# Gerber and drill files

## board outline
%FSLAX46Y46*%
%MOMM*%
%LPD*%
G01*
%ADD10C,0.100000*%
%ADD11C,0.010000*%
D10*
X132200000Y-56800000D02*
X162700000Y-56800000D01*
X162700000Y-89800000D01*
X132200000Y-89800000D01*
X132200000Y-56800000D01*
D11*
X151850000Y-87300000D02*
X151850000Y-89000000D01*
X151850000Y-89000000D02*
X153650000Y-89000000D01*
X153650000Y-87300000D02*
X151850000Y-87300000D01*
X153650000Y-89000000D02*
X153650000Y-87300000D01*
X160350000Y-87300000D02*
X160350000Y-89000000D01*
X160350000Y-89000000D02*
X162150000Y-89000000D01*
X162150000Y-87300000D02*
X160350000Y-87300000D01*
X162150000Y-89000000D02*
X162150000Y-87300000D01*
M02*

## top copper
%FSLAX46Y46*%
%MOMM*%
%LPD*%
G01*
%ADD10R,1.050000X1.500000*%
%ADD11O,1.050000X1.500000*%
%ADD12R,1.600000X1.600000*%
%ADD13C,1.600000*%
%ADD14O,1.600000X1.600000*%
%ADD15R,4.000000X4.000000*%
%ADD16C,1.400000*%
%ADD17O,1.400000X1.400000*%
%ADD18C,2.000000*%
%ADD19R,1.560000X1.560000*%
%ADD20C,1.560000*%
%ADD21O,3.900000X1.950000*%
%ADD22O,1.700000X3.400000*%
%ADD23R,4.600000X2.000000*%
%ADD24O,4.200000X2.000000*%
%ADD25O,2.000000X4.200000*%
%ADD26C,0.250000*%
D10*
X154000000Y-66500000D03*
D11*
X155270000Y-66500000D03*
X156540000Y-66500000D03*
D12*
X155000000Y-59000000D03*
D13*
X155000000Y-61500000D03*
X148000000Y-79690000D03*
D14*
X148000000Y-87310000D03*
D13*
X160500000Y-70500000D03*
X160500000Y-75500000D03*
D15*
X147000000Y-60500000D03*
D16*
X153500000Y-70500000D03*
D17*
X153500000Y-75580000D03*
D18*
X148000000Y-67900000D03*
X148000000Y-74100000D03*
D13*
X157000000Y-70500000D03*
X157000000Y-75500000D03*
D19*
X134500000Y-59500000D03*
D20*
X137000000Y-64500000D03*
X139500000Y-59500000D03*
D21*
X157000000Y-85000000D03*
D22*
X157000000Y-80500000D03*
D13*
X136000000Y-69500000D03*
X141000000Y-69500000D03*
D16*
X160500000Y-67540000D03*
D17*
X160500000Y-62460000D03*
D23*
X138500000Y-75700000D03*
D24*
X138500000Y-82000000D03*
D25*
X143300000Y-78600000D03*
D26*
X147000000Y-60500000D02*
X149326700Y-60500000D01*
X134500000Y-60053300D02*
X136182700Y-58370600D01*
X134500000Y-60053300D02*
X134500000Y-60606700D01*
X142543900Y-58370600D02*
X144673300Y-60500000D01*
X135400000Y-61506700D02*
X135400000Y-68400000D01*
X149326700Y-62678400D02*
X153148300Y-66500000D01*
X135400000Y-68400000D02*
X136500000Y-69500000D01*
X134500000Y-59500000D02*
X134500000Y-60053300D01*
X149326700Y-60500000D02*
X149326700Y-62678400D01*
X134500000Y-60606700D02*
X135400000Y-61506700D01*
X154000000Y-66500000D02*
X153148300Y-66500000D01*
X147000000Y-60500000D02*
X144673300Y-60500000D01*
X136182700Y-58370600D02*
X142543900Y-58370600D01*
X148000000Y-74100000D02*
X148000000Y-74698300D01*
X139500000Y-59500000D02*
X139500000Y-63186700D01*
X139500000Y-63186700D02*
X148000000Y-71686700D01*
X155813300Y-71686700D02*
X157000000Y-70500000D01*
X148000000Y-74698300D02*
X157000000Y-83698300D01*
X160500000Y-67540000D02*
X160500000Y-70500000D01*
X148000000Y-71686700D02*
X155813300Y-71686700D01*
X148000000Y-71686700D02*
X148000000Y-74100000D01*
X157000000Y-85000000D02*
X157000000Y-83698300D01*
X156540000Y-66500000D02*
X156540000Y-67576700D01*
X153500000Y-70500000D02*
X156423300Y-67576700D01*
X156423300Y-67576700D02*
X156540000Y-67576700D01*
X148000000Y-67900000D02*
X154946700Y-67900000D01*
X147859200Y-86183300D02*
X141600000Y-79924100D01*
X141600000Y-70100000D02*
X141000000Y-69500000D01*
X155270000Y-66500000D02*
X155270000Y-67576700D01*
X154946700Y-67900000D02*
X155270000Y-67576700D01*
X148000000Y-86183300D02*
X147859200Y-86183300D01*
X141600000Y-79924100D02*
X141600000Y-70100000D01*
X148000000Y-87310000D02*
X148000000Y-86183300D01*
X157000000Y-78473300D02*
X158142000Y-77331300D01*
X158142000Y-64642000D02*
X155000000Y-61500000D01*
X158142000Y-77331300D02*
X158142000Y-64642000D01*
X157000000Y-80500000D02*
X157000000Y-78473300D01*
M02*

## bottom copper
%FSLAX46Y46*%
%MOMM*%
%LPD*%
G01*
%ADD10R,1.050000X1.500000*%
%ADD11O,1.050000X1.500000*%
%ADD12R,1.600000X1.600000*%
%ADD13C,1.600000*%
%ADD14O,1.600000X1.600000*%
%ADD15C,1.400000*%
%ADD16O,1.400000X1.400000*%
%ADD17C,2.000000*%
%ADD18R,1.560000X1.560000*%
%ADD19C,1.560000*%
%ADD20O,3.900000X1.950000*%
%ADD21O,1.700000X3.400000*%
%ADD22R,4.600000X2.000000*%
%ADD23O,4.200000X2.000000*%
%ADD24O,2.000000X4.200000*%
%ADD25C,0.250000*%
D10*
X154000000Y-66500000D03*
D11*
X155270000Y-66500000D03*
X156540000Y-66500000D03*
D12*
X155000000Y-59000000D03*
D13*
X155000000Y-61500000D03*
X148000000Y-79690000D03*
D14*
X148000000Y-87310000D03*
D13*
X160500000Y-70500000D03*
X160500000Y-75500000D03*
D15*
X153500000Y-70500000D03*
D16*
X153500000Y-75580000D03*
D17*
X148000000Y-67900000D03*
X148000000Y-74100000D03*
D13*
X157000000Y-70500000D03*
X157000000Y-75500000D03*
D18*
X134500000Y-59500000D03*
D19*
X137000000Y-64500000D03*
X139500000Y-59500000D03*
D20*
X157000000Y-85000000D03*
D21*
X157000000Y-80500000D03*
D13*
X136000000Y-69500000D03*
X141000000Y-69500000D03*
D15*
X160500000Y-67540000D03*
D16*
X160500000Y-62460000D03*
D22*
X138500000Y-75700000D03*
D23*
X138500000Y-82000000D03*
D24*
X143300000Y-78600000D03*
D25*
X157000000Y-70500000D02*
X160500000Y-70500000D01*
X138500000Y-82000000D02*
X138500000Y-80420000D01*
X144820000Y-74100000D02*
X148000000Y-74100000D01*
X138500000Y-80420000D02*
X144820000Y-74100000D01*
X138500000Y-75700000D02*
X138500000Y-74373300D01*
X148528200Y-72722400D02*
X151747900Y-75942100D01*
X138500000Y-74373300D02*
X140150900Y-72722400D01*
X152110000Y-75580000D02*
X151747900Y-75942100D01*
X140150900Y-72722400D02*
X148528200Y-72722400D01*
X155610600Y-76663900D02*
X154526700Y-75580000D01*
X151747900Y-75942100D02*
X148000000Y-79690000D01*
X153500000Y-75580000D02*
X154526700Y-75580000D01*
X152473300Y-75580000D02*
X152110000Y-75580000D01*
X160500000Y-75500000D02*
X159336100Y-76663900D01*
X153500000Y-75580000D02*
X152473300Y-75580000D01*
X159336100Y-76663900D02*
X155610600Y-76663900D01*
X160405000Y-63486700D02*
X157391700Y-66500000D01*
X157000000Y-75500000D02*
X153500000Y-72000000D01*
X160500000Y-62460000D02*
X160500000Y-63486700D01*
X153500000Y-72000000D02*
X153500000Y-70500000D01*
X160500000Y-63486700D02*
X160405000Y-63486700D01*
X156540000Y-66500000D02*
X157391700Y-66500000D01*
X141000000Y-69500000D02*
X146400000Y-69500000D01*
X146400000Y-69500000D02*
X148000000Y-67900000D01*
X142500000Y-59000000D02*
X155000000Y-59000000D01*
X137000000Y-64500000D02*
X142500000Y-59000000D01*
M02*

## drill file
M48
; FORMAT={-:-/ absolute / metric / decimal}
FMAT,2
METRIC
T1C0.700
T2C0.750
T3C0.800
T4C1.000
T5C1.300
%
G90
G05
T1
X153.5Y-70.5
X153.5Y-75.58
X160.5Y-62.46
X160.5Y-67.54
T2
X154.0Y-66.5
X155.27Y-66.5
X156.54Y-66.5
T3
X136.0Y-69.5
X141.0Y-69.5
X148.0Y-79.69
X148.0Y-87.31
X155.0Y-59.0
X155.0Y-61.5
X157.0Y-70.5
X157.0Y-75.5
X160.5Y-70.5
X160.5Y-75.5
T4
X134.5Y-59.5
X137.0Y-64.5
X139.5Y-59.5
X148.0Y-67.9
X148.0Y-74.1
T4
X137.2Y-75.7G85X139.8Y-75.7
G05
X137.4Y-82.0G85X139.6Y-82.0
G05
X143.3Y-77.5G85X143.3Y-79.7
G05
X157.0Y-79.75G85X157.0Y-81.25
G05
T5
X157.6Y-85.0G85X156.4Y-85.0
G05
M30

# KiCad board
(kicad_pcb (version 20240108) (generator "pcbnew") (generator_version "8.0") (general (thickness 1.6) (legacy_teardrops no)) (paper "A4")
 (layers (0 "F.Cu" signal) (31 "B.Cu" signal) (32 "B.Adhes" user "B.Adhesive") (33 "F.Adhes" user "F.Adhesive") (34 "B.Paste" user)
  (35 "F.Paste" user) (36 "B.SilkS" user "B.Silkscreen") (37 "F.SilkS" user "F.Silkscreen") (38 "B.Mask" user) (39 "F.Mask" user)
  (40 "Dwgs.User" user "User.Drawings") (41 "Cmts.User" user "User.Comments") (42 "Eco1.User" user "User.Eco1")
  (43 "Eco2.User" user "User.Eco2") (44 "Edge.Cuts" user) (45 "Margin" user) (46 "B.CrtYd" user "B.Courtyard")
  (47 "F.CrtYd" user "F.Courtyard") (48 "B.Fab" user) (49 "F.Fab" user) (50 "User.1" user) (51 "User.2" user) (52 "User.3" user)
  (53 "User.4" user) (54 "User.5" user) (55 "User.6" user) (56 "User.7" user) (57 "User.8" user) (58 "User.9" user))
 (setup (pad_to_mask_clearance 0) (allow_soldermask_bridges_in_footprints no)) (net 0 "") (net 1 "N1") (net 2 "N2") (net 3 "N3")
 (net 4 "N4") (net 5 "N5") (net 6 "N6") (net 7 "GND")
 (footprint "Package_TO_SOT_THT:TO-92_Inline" (layer "F.Cu") (at 154 66.5)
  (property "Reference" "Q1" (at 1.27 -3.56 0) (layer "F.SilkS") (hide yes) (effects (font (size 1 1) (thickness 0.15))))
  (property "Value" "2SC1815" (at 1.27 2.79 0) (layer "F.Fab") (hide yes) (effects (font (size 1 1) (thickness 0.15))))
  (pad "1" thru_hole rect (at 0 0) (size 1.05 1.5) (drill 0.75) (layers "*.Cu" "*.Mask") (remove_unused_layers no) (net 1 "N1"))
  (pad "2" thru_hole oval (at 1.27 0) (size 1.05 1.5) (drill 0.75) (layers "*.Cu" "*.Mask") (remove_unused_layers no) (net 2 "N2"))
  (pad "3" thru_hole oval (at 2.54 0) (size 1.05 1.5) (drill 0.75) (layers "*.Cu" "*.Mask") (remove_unused_layers no) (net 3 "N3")))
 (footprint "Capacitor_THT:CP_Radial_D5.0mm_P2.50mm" (layer "F.Cu") (at 155 59 -90)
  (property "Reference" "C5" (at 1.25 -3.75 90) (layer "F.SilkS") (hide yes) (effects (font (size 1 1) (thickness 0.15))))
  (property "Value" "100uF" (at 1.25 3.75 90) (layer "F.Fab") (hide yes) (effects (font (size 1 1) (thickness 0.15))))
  (pad "1" thru_hole rect (at 0 0 270) (size 1.6 1.6) (drill 0.8) (layers "*.Cu" "*.Mask") (remove_unused_layers no) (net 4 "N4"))
  (pad "2" thru_hole circle (at 2.5 0 270) (size 1.6 1.6) (drill 0.8) (layers "*.Cu" "*.Mask") (remove_unused_layers no) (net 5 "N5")))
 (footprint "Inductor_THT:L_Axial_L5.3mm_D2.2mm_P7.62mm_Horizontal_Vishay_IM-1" (layer "F.Cu") (at 148 79.69 -90)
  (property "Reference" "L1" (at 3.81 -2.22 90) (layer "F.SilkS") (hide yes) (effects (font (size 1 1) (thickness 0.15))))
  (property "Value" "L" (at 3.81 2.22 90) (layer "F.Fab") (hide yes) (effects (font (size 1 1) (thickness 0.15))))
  (pad "1" thru_hole circle (at 0 0 270) (size 1.6 1.6) (drill 0.8) (layers "*.Cu" "*.Mask") (remove_unused_layers no) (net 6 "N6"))
  (pad "2" thru_hole oval (at 7.62 0 270) (size 1.6 1.6) (drill 0.8) (layers "*.Cu" "*.Mask") (remove_unused_layers no) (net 2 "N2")))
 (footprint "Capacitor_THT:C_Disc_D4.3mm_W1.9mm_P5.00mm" (layer "F.Cu") (at 160.5 70.5 -90)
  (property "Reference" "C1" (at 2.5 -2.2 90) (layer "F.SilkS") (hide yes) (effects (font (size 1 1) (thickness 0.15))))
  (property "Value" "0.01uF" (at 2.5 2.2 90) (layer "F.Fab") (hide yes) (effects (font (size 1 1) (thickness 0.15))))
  (pad "1" thru_hole circle (at 0 0 270) (size 1.6 1.6) (drill 0.8) (layers "*.Cu" "*.Mask") (remove_unused_layers no) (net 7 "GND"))
  (pad "2" thru_hole circle (at 5 0 270) (size 1.6 1.6) (drill 0.8) (layers "*.Cu" "*.Mask") (remove_unused_layers no) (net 6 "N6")))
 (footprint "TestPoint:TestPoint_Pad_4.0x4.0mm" (layer "F.Cu") (at 147 60.5)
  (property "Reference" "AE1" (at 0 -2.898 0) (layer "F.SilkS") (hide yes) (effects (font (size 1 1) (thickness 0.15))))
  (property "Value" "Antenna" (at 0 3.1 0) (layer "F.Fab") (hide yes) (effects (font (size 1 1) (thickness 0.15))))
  (pad "1" smd rect (at 0 0) (size 4 4) (layers "F.Cu" "F.Mask") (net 1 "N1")))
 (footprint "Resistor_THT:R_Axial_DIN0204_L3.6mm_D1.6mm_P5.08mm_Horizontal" (layer "F.Cu") (at 153.5 70.5 -90)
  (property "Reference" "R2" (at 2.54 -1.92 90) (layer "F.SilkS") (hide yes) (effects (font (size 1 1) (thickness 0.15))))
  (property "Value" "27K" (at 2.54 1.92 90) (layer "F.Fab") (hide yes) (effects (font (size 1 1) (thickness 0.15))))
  (pad "1" thru_hole circle (at 0 0 270) (size 1.4 1.4) (drill 0.7) (layers "*.Cu" "*.Mask") (remove_unused_layers no) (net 3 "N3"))
  (pad "2" thru_hole oval (at 5.08 0 270) (size 1.4 1.4) (drill 0.7) (layers "*.Cu" "*.Mask") (remove_unused_layers no) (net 6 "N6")))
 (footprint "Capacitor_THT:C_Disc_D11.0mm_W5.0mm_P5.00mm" (layer "F.Cu") (at 148 68.4 -90)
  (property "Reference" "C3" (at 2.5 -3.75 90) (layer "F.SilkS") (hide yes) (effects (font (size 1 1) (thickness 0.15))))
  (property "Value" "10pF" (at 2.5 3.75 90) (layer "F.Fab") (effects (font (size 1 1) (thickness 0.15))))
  (pad "1" thru_hole circle (at -0.5 0 270) (size 2 2) (drill 1) (layers "*.Cu" "*.Mask") (remove_unused_layers no) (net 2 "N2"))
  (pad "2" thru_hole circle (at 5.7 0 270) (size 2 2) (drill 1) (layers "*.Cu" "*.Mask") (remove_unused_layers no) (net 7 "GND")))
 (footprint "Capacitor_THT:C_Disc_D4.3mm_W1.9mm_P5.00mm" (layer "F.Cu") (at 157 70.5 -90)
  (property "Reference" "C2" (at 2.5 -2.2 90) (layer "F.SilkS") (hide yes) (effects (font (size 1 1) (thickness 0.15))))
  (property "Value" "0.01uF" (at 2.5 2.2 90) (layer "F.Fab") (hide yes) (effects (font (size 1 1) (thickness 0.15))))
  (pad "1" thru_hole circle (at 0 0 270) (size 1.6 1.6) (drill 0.8) (layers "*.Cu" "*.Mask") (remove_unused_layers no) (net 7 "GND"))
  (pad "2" thru_hole circle (at 5 0 270) (size 1.6 1.6) (drill 0.8) (layers "*.Cu" "*.Mask") (remove_unused_layers no) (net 3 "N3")))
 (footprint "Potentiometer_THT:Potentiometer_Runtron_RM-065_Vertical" (layer "F.Cu") (at 134.5 59.5)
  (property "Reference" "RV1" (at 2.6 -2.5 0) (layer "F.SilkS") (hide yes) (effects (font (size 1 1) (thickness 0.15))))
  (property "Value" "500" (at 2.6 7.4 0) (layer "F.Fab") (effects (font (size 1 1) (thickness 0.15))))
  (pad "1" thru_hole rect (at 0 0) (size 1.56 1.56) (drill 1) (layers "*.Cu" "*.Mask") (remove_unused_layers no) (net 1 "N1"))
  (pad "2" thru_hole circle (at 2.5 5) (size 1.56 1.56) (drill 1) (layers "*.Cu" "*.Mask") (remove_unused_layers no) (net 4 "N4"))
  (pad "3" thru_hole circle (at 5 0) (size 1.56 1.56) (drill 1) (layers "*.Cu" "*.Mask") (remove_unused_layers no) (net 7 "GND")))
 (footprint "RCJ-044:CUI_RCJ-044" (layer "F.Cu") (at 157 85 -90)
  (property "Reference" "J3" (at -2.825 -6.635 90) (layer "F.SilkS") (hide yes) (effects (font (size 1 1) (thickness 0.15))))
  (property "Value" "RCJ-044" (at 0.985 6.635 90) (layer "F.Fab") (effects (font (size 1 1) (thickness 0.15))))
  (fp_line (start 2.3 5.15) (end 4 5.15) (stroke (width 0.01) (type solid)) (layer "Edge.Cuts"))
  (fp_line (start 4 5.15) (end 4 3.35) (stroke (width 0.01) (type solid)) (layer "Edge.Cuts"))
  (fp_line (start 2.3 3.35) (end 2.3 5.15) (stroke (width 0.01) (type solid)) (layer "Edge.Cuts"))
  (fp_line (start 4 3.35) (end 2.3 3.35) (stroke (width 0.01) (type solid)) (layer "Edge.Cuts"))
  (fp_line (start 2.3 -3.35) (end 4 -3.35) (stroke (width 0.01) (type solid)) (layer "Edge.Cuts"))
  (fp_line (start 4 -3.35) (end 4 -5.15) (stroke (width 0.01) (type solid)) (layer "Edge.Cuts"))
  (fp_line (start 2.3 -5.15) (end 2.3 -3.35) (stroke (width 0.01) (type solid)) (layer "Edge.Cuts"))
  (fp_line (start 4 -5.15) (end 2.3 -5.15) (stroke (width 0.01) (type solid)) (layer "Edge.Cuts"))
  (pad "1" thru_hole oval (at 0 0 270) (size 1.95 3.9) (drill oval 1.3 2.5) (layers "*.Cu" "*.Mask") (remove_unused_layers no) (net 7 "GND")
   (solder_mask_margin 0.102))
  (pad "2" thru_hole oval (at -4.5 0 270) (size 3.4 1.7) (drill oval 2.5 1) (layers "*.Cu" "*.Mask") (remove_unused_layers no) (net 5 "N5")
   (solder_mask_margin 0.102)))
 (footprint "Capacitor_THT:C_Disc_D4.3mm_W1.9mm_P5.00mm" (layer "F.Cu") (at 136 69.5)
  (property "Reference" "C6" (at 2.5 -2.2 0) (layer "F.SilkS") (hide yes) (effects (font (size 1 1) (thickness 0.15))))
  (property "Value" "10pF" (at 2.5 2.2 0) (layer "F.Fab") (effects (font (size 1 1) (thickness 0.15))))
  (pad "1" thru_hole circle (at 0 0) (size 1.6 1.6) (drill 0.8) (layers "*.Cu" "*.Mask") (remove_unused_layers no) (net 1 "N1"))
  (pad "2" thru_hole circle (at 5 0) (size 1.6 1.6) (drill 0.8) (layers "*.Cu" "*.Mask") (remove_unused_layers no) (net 2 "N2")))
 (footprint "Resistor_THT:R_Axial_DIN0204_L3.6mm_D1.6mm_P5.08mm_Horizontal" (layer "F.Cu") (at 160.5 67.54 90)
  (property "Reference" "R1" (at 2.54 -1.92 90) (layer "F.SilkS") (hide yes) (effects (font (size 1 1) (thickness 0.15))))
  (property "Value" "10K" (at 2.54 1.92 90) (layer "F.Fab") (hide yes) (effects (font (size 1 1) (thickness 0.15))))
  (pad "1" thru_hole circle (at 0 0 90) (size 1.4 1.4) (drill 0.7) (layers "*.Cu" "*.Mask") (remove_unused_layers no) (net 7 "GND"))
  (pad "2" thru_hole oval (at 5.08 0 90) (size 1.4 1.4) (drill 0.7) (layers "*.Cu" "*.Mask") (remove_unused_layers no) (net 3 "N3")))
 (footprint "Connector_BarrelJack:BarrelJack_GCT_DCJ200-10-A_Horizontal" (layer "F.Cu") (at 138.5 75.7)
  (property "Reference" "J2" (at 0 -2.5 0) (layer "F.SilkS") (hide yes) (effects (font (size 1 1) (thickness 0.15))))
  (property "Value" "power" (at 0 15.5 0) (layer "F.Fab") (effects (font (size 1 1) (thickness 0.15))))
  (pad "1" thru_hole rect (at 0 0) (size 4.6 2) (drill oval 3.6 1) (layers "*.Cu" "*.Mask") (remove_unused_layers no) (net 6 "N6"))
  (pad "2" thru_hole oval (at 0 6.3) (size 4.2 2) (drill oval 3.2 1) (layers "*.Cu" "*.Mask") (remove_unused_layers no) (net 7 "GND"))
  (pad "3" thru_hole oval (at 4.8 2.9) (size 2 4.2) (drill oval 1 3.2) (layers "*.Cu" "*.Mask") (remove_unused_layers no)))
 (gr_rect (start 132.2 56.8) (end 162.7 89.8) (stroke (width 0.1) (type solid)) (fill none) (layer "Edge.Cuts"))
 (segment (start 147 60.5) (end 149.3267 60.5) (width 0.25) (layer "F.Cu") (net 1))
 (segment (start 134.5 60.0533) (end 136.1827 58.3706) (width 0.25) (layer "F.Cu") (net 1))
 (segment (start 134.5 60.0533) (end 134.5 60.6067) (width 0.25) (layer "F.Cu") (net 1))
 (segment (start 142.5439 58.3706) (end 144.6733 60.5) (width 0.25) (layer "F.Cu") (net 1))
 (segment (start 135.4 61.5067) (end 135.4 68.4) (width 0.25) (layer "F.Cu") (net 1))
 (segment (start 149.3267 62.6784) (end 153.1483 66.5) (width 0.25) (layer "F.Cu") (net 1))
 (segment (start 135.4 68.4) (end 136.5 69.5) (width 0.25) (layer "F.Cu") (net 1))
 (segment (start 134.5 59.5) (end 134.5 60.0533) (width 0.25) (layer "F.Cu") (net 1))
 (segment (start 149.3267 60.5) (end 149.3267 62.6784) (width 0.25) (layer "F.Cu") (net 1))
 (segment (start 134.5 60.6067) (end 135.4 61.5067) (width 0.25) (layer "F.Cu") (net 1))
 (segment (start 154 66.5) (end 153.1483 66.5) (width 0.25) (layer "F.Cu") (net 1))
 (segment (start 147 60.5) (end 144.6733 60.5) (width 0.25) (layer "F.Cu") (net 1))
 (segment (start 136.1827 58.3706) (end 142.5439 58.3706) (width 0.25) (layer "F.Cu") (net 1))
 (segment (start 148 74.1) (end 148 74.6983) (width 0.25) (layer "F.Cu") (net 7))
 (segment (start 139.5 59.5) (end 139.5 63.1867) (width 0.25) (layer "F.Cu") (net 7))
 (segment (start 139.5 63.1867) (end 148 71.6867) (width 0.25) (layer "F.Cu") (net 7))
 (segment (start 155.8133 71.6867) (end 157 70.5) (width 0.25) (layer "F.Cu") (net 7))
 (segment (start 148 74.6983) (end 157 83.6983) (width 0.25) (layer "F.Cu") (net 7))
 (segment (start 160.5 67.54) (end 160.5 70.5) (width 0.25) (layer "F.Cu") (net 7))
 (segment (start 148 71.6867) (end 155.8133 71.6867) (width 0.25) (layer "F.Cu") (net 7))
 (segment (start 148 71.6867) (end 148 74.1) (width 0.25) (layer "F.Cu") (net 7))
 (segment (start 157 85) (end 157 83.6983) (width 0.25) (layer "F.Cu") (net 7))
 (segment (start 157 70.5) (end 160.5 70.5) (width 0.25) (layer "B.Cu") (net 7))
 (segment (start 138.5 82) (end 138.5 80.42) (width 0.25) (layer "B.Cu") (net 7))
 (segment (start 144.82 74.1) (end 148 74.1) (width 0.25) (layer "B.Cu") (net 7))
 (segment (start 138.5 80.42) (end 144.82 74.1) (width 0.25) (layer "B.Cu") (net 7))
 (segment (start 138.5 75.7) (end 138.5 74.3733) (width 0.25) (layer "B.Cu") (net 6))
 (segment (start 148.5282 72.7224) (end 151.7479 75.9421) (width 0.25) (layer "B.Cu") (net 6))
 (segment (start 138.5 74.3733) (end 140.1509 72.7224) (width 0.25) (layer "B.Cu") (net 6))
 (segment (start 152.11 75.58) (end 151.7479 75.9421) (width 0.25) (layer "B.Cu") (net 6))
 (segment (start 140.1509 72.7224) (end 148.5282 72.7224) (width 0.25) (layer "B.Cu") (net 6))
 (segment (start 155.6106 76.6639) (end 154.5267 75.58) (width 0.25) (layer "B.Cu") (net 6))
 (segment (start 151.7479 75.9421) (end 148 79.69) (width 0.25) (layer "B.Cu") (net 6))
 (segment (start 153.5 75.58) (end 154.5267 75.58) (width 0.25) (layer "B.Cu") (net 6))
 (segment (start 152.4733 75.58) (end 152.11 75.58) (width 0.25) (layer "B.Cu") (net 6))
 (segment (start 160.5 75.5) (end 159.3361 76.6639) (width 0.25) (layer "B.Cu") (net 6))
 (segment (start 153.5 75.58) (end 152.4733 75.58) (width 0.25) (layer "B.Cu") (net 6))
 (segment (start 159.3361 76.6639) (end 155.6106 76.6639) (width 0.25) (layer "B.Cu") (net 6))
 (segment (start 156.54 66.5) (end 156.54 67.5767) (width 0.25) (layer "F.Cu") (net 3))
 (segment (start 153.5 70.5) (end 156.4233 67.5767) (width 0.25) (layer "F.Cu") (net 3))
 (segment (start 156.4233 67.5767) (end 156.54 67.5767) (width 0.25) (layer "F.Cu") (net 3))
 (segment (start 160.405 63.4867) (end 157.3917 66.5) (width 0.25) (layer "B.Cu") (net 3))
 (segment (start 157 75.5) (end 153.5 72) (width 0.25) (layer "B.Cu") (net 3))
 (segment (start 160.5 62.46) (end 160.5 63.4867) (width 0.25) (layer "B.Cu") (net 3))
 (segment (start 153.5 72) (end 153.5 70.5) (width 0.25) (layer "B.Cu") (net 3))
 (segment (start 160.5 63.4867) (end 160.405 63.4867) (width 0.25) (layer "B.Cu") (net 3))
 (segment (start 156.54 66.5) (end 157.3917 66.5) (width 0.25) (layer "B.Cu") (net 3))
 (segment (start 148 67.9) (end 154.9467 67.9) (width 0.25) (layer "F.Cu") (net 2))
 (segment (start 147.8592 86.1833) (end 141.6 79.9241) (width 0.25) (layer "F.Cu") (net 2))
 (segment (start 141.6 70.1) (end 141 69.5) (width 0.25) (layer "F.Cu") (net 2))
 (segment (start 155.27 66.5) (end 155.27 67.5767) (width 0.25) (layer "F.Cu") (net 2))
 (segment (start 154.9467 67.9) (end 155.27 67.5767) (width 0.25) (layer "F.Cu") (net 2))
 (segment (start 148 86.1833) (end 147.8592 86.1833) (width 0.25) (layer "F.Cu") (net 2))
 (segment (start 141.6 79.9241) (end 141.6 70.1) (width 0.25) (layer "F.Cu") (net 2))
 (segment (start 148 87.31) (end 148 86.1833) (width 0.25) (layer "F.Cu") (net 2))
 (segment (start 141 69.5) (end 146.4 69.5) (width 0.25) (layer "B.Cu") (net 2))
 (segment (start 146.4 69.5) (end 148 67.9) (width 0.25) (layer "B.Cu") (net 2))
 (segment (start 157 78.4733) (end 158.142 77.3313) (width 0.25) (layer "F.Cu") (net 5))
 (segment (start 158.142 64.642) (end 155 61.5) (width 0.25) (layer "F.Cu") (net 5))
 (segment (start 158.142 77.3313) (end 158.142 64.642) (width 0.25) (layer "F.Cu") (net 5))
 (segment (start 157 80.5) (end 157 78.4733) (width 0.25) (layer "F.Cu") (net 5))
 (segment (start 142.5 59) (end 155 59) (width 0.25) (layer "B.Cu") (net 4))
 (segment (start 137 64.5) (end 142.5 59) (width 0.25) (layer "B.Cu") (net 4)))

